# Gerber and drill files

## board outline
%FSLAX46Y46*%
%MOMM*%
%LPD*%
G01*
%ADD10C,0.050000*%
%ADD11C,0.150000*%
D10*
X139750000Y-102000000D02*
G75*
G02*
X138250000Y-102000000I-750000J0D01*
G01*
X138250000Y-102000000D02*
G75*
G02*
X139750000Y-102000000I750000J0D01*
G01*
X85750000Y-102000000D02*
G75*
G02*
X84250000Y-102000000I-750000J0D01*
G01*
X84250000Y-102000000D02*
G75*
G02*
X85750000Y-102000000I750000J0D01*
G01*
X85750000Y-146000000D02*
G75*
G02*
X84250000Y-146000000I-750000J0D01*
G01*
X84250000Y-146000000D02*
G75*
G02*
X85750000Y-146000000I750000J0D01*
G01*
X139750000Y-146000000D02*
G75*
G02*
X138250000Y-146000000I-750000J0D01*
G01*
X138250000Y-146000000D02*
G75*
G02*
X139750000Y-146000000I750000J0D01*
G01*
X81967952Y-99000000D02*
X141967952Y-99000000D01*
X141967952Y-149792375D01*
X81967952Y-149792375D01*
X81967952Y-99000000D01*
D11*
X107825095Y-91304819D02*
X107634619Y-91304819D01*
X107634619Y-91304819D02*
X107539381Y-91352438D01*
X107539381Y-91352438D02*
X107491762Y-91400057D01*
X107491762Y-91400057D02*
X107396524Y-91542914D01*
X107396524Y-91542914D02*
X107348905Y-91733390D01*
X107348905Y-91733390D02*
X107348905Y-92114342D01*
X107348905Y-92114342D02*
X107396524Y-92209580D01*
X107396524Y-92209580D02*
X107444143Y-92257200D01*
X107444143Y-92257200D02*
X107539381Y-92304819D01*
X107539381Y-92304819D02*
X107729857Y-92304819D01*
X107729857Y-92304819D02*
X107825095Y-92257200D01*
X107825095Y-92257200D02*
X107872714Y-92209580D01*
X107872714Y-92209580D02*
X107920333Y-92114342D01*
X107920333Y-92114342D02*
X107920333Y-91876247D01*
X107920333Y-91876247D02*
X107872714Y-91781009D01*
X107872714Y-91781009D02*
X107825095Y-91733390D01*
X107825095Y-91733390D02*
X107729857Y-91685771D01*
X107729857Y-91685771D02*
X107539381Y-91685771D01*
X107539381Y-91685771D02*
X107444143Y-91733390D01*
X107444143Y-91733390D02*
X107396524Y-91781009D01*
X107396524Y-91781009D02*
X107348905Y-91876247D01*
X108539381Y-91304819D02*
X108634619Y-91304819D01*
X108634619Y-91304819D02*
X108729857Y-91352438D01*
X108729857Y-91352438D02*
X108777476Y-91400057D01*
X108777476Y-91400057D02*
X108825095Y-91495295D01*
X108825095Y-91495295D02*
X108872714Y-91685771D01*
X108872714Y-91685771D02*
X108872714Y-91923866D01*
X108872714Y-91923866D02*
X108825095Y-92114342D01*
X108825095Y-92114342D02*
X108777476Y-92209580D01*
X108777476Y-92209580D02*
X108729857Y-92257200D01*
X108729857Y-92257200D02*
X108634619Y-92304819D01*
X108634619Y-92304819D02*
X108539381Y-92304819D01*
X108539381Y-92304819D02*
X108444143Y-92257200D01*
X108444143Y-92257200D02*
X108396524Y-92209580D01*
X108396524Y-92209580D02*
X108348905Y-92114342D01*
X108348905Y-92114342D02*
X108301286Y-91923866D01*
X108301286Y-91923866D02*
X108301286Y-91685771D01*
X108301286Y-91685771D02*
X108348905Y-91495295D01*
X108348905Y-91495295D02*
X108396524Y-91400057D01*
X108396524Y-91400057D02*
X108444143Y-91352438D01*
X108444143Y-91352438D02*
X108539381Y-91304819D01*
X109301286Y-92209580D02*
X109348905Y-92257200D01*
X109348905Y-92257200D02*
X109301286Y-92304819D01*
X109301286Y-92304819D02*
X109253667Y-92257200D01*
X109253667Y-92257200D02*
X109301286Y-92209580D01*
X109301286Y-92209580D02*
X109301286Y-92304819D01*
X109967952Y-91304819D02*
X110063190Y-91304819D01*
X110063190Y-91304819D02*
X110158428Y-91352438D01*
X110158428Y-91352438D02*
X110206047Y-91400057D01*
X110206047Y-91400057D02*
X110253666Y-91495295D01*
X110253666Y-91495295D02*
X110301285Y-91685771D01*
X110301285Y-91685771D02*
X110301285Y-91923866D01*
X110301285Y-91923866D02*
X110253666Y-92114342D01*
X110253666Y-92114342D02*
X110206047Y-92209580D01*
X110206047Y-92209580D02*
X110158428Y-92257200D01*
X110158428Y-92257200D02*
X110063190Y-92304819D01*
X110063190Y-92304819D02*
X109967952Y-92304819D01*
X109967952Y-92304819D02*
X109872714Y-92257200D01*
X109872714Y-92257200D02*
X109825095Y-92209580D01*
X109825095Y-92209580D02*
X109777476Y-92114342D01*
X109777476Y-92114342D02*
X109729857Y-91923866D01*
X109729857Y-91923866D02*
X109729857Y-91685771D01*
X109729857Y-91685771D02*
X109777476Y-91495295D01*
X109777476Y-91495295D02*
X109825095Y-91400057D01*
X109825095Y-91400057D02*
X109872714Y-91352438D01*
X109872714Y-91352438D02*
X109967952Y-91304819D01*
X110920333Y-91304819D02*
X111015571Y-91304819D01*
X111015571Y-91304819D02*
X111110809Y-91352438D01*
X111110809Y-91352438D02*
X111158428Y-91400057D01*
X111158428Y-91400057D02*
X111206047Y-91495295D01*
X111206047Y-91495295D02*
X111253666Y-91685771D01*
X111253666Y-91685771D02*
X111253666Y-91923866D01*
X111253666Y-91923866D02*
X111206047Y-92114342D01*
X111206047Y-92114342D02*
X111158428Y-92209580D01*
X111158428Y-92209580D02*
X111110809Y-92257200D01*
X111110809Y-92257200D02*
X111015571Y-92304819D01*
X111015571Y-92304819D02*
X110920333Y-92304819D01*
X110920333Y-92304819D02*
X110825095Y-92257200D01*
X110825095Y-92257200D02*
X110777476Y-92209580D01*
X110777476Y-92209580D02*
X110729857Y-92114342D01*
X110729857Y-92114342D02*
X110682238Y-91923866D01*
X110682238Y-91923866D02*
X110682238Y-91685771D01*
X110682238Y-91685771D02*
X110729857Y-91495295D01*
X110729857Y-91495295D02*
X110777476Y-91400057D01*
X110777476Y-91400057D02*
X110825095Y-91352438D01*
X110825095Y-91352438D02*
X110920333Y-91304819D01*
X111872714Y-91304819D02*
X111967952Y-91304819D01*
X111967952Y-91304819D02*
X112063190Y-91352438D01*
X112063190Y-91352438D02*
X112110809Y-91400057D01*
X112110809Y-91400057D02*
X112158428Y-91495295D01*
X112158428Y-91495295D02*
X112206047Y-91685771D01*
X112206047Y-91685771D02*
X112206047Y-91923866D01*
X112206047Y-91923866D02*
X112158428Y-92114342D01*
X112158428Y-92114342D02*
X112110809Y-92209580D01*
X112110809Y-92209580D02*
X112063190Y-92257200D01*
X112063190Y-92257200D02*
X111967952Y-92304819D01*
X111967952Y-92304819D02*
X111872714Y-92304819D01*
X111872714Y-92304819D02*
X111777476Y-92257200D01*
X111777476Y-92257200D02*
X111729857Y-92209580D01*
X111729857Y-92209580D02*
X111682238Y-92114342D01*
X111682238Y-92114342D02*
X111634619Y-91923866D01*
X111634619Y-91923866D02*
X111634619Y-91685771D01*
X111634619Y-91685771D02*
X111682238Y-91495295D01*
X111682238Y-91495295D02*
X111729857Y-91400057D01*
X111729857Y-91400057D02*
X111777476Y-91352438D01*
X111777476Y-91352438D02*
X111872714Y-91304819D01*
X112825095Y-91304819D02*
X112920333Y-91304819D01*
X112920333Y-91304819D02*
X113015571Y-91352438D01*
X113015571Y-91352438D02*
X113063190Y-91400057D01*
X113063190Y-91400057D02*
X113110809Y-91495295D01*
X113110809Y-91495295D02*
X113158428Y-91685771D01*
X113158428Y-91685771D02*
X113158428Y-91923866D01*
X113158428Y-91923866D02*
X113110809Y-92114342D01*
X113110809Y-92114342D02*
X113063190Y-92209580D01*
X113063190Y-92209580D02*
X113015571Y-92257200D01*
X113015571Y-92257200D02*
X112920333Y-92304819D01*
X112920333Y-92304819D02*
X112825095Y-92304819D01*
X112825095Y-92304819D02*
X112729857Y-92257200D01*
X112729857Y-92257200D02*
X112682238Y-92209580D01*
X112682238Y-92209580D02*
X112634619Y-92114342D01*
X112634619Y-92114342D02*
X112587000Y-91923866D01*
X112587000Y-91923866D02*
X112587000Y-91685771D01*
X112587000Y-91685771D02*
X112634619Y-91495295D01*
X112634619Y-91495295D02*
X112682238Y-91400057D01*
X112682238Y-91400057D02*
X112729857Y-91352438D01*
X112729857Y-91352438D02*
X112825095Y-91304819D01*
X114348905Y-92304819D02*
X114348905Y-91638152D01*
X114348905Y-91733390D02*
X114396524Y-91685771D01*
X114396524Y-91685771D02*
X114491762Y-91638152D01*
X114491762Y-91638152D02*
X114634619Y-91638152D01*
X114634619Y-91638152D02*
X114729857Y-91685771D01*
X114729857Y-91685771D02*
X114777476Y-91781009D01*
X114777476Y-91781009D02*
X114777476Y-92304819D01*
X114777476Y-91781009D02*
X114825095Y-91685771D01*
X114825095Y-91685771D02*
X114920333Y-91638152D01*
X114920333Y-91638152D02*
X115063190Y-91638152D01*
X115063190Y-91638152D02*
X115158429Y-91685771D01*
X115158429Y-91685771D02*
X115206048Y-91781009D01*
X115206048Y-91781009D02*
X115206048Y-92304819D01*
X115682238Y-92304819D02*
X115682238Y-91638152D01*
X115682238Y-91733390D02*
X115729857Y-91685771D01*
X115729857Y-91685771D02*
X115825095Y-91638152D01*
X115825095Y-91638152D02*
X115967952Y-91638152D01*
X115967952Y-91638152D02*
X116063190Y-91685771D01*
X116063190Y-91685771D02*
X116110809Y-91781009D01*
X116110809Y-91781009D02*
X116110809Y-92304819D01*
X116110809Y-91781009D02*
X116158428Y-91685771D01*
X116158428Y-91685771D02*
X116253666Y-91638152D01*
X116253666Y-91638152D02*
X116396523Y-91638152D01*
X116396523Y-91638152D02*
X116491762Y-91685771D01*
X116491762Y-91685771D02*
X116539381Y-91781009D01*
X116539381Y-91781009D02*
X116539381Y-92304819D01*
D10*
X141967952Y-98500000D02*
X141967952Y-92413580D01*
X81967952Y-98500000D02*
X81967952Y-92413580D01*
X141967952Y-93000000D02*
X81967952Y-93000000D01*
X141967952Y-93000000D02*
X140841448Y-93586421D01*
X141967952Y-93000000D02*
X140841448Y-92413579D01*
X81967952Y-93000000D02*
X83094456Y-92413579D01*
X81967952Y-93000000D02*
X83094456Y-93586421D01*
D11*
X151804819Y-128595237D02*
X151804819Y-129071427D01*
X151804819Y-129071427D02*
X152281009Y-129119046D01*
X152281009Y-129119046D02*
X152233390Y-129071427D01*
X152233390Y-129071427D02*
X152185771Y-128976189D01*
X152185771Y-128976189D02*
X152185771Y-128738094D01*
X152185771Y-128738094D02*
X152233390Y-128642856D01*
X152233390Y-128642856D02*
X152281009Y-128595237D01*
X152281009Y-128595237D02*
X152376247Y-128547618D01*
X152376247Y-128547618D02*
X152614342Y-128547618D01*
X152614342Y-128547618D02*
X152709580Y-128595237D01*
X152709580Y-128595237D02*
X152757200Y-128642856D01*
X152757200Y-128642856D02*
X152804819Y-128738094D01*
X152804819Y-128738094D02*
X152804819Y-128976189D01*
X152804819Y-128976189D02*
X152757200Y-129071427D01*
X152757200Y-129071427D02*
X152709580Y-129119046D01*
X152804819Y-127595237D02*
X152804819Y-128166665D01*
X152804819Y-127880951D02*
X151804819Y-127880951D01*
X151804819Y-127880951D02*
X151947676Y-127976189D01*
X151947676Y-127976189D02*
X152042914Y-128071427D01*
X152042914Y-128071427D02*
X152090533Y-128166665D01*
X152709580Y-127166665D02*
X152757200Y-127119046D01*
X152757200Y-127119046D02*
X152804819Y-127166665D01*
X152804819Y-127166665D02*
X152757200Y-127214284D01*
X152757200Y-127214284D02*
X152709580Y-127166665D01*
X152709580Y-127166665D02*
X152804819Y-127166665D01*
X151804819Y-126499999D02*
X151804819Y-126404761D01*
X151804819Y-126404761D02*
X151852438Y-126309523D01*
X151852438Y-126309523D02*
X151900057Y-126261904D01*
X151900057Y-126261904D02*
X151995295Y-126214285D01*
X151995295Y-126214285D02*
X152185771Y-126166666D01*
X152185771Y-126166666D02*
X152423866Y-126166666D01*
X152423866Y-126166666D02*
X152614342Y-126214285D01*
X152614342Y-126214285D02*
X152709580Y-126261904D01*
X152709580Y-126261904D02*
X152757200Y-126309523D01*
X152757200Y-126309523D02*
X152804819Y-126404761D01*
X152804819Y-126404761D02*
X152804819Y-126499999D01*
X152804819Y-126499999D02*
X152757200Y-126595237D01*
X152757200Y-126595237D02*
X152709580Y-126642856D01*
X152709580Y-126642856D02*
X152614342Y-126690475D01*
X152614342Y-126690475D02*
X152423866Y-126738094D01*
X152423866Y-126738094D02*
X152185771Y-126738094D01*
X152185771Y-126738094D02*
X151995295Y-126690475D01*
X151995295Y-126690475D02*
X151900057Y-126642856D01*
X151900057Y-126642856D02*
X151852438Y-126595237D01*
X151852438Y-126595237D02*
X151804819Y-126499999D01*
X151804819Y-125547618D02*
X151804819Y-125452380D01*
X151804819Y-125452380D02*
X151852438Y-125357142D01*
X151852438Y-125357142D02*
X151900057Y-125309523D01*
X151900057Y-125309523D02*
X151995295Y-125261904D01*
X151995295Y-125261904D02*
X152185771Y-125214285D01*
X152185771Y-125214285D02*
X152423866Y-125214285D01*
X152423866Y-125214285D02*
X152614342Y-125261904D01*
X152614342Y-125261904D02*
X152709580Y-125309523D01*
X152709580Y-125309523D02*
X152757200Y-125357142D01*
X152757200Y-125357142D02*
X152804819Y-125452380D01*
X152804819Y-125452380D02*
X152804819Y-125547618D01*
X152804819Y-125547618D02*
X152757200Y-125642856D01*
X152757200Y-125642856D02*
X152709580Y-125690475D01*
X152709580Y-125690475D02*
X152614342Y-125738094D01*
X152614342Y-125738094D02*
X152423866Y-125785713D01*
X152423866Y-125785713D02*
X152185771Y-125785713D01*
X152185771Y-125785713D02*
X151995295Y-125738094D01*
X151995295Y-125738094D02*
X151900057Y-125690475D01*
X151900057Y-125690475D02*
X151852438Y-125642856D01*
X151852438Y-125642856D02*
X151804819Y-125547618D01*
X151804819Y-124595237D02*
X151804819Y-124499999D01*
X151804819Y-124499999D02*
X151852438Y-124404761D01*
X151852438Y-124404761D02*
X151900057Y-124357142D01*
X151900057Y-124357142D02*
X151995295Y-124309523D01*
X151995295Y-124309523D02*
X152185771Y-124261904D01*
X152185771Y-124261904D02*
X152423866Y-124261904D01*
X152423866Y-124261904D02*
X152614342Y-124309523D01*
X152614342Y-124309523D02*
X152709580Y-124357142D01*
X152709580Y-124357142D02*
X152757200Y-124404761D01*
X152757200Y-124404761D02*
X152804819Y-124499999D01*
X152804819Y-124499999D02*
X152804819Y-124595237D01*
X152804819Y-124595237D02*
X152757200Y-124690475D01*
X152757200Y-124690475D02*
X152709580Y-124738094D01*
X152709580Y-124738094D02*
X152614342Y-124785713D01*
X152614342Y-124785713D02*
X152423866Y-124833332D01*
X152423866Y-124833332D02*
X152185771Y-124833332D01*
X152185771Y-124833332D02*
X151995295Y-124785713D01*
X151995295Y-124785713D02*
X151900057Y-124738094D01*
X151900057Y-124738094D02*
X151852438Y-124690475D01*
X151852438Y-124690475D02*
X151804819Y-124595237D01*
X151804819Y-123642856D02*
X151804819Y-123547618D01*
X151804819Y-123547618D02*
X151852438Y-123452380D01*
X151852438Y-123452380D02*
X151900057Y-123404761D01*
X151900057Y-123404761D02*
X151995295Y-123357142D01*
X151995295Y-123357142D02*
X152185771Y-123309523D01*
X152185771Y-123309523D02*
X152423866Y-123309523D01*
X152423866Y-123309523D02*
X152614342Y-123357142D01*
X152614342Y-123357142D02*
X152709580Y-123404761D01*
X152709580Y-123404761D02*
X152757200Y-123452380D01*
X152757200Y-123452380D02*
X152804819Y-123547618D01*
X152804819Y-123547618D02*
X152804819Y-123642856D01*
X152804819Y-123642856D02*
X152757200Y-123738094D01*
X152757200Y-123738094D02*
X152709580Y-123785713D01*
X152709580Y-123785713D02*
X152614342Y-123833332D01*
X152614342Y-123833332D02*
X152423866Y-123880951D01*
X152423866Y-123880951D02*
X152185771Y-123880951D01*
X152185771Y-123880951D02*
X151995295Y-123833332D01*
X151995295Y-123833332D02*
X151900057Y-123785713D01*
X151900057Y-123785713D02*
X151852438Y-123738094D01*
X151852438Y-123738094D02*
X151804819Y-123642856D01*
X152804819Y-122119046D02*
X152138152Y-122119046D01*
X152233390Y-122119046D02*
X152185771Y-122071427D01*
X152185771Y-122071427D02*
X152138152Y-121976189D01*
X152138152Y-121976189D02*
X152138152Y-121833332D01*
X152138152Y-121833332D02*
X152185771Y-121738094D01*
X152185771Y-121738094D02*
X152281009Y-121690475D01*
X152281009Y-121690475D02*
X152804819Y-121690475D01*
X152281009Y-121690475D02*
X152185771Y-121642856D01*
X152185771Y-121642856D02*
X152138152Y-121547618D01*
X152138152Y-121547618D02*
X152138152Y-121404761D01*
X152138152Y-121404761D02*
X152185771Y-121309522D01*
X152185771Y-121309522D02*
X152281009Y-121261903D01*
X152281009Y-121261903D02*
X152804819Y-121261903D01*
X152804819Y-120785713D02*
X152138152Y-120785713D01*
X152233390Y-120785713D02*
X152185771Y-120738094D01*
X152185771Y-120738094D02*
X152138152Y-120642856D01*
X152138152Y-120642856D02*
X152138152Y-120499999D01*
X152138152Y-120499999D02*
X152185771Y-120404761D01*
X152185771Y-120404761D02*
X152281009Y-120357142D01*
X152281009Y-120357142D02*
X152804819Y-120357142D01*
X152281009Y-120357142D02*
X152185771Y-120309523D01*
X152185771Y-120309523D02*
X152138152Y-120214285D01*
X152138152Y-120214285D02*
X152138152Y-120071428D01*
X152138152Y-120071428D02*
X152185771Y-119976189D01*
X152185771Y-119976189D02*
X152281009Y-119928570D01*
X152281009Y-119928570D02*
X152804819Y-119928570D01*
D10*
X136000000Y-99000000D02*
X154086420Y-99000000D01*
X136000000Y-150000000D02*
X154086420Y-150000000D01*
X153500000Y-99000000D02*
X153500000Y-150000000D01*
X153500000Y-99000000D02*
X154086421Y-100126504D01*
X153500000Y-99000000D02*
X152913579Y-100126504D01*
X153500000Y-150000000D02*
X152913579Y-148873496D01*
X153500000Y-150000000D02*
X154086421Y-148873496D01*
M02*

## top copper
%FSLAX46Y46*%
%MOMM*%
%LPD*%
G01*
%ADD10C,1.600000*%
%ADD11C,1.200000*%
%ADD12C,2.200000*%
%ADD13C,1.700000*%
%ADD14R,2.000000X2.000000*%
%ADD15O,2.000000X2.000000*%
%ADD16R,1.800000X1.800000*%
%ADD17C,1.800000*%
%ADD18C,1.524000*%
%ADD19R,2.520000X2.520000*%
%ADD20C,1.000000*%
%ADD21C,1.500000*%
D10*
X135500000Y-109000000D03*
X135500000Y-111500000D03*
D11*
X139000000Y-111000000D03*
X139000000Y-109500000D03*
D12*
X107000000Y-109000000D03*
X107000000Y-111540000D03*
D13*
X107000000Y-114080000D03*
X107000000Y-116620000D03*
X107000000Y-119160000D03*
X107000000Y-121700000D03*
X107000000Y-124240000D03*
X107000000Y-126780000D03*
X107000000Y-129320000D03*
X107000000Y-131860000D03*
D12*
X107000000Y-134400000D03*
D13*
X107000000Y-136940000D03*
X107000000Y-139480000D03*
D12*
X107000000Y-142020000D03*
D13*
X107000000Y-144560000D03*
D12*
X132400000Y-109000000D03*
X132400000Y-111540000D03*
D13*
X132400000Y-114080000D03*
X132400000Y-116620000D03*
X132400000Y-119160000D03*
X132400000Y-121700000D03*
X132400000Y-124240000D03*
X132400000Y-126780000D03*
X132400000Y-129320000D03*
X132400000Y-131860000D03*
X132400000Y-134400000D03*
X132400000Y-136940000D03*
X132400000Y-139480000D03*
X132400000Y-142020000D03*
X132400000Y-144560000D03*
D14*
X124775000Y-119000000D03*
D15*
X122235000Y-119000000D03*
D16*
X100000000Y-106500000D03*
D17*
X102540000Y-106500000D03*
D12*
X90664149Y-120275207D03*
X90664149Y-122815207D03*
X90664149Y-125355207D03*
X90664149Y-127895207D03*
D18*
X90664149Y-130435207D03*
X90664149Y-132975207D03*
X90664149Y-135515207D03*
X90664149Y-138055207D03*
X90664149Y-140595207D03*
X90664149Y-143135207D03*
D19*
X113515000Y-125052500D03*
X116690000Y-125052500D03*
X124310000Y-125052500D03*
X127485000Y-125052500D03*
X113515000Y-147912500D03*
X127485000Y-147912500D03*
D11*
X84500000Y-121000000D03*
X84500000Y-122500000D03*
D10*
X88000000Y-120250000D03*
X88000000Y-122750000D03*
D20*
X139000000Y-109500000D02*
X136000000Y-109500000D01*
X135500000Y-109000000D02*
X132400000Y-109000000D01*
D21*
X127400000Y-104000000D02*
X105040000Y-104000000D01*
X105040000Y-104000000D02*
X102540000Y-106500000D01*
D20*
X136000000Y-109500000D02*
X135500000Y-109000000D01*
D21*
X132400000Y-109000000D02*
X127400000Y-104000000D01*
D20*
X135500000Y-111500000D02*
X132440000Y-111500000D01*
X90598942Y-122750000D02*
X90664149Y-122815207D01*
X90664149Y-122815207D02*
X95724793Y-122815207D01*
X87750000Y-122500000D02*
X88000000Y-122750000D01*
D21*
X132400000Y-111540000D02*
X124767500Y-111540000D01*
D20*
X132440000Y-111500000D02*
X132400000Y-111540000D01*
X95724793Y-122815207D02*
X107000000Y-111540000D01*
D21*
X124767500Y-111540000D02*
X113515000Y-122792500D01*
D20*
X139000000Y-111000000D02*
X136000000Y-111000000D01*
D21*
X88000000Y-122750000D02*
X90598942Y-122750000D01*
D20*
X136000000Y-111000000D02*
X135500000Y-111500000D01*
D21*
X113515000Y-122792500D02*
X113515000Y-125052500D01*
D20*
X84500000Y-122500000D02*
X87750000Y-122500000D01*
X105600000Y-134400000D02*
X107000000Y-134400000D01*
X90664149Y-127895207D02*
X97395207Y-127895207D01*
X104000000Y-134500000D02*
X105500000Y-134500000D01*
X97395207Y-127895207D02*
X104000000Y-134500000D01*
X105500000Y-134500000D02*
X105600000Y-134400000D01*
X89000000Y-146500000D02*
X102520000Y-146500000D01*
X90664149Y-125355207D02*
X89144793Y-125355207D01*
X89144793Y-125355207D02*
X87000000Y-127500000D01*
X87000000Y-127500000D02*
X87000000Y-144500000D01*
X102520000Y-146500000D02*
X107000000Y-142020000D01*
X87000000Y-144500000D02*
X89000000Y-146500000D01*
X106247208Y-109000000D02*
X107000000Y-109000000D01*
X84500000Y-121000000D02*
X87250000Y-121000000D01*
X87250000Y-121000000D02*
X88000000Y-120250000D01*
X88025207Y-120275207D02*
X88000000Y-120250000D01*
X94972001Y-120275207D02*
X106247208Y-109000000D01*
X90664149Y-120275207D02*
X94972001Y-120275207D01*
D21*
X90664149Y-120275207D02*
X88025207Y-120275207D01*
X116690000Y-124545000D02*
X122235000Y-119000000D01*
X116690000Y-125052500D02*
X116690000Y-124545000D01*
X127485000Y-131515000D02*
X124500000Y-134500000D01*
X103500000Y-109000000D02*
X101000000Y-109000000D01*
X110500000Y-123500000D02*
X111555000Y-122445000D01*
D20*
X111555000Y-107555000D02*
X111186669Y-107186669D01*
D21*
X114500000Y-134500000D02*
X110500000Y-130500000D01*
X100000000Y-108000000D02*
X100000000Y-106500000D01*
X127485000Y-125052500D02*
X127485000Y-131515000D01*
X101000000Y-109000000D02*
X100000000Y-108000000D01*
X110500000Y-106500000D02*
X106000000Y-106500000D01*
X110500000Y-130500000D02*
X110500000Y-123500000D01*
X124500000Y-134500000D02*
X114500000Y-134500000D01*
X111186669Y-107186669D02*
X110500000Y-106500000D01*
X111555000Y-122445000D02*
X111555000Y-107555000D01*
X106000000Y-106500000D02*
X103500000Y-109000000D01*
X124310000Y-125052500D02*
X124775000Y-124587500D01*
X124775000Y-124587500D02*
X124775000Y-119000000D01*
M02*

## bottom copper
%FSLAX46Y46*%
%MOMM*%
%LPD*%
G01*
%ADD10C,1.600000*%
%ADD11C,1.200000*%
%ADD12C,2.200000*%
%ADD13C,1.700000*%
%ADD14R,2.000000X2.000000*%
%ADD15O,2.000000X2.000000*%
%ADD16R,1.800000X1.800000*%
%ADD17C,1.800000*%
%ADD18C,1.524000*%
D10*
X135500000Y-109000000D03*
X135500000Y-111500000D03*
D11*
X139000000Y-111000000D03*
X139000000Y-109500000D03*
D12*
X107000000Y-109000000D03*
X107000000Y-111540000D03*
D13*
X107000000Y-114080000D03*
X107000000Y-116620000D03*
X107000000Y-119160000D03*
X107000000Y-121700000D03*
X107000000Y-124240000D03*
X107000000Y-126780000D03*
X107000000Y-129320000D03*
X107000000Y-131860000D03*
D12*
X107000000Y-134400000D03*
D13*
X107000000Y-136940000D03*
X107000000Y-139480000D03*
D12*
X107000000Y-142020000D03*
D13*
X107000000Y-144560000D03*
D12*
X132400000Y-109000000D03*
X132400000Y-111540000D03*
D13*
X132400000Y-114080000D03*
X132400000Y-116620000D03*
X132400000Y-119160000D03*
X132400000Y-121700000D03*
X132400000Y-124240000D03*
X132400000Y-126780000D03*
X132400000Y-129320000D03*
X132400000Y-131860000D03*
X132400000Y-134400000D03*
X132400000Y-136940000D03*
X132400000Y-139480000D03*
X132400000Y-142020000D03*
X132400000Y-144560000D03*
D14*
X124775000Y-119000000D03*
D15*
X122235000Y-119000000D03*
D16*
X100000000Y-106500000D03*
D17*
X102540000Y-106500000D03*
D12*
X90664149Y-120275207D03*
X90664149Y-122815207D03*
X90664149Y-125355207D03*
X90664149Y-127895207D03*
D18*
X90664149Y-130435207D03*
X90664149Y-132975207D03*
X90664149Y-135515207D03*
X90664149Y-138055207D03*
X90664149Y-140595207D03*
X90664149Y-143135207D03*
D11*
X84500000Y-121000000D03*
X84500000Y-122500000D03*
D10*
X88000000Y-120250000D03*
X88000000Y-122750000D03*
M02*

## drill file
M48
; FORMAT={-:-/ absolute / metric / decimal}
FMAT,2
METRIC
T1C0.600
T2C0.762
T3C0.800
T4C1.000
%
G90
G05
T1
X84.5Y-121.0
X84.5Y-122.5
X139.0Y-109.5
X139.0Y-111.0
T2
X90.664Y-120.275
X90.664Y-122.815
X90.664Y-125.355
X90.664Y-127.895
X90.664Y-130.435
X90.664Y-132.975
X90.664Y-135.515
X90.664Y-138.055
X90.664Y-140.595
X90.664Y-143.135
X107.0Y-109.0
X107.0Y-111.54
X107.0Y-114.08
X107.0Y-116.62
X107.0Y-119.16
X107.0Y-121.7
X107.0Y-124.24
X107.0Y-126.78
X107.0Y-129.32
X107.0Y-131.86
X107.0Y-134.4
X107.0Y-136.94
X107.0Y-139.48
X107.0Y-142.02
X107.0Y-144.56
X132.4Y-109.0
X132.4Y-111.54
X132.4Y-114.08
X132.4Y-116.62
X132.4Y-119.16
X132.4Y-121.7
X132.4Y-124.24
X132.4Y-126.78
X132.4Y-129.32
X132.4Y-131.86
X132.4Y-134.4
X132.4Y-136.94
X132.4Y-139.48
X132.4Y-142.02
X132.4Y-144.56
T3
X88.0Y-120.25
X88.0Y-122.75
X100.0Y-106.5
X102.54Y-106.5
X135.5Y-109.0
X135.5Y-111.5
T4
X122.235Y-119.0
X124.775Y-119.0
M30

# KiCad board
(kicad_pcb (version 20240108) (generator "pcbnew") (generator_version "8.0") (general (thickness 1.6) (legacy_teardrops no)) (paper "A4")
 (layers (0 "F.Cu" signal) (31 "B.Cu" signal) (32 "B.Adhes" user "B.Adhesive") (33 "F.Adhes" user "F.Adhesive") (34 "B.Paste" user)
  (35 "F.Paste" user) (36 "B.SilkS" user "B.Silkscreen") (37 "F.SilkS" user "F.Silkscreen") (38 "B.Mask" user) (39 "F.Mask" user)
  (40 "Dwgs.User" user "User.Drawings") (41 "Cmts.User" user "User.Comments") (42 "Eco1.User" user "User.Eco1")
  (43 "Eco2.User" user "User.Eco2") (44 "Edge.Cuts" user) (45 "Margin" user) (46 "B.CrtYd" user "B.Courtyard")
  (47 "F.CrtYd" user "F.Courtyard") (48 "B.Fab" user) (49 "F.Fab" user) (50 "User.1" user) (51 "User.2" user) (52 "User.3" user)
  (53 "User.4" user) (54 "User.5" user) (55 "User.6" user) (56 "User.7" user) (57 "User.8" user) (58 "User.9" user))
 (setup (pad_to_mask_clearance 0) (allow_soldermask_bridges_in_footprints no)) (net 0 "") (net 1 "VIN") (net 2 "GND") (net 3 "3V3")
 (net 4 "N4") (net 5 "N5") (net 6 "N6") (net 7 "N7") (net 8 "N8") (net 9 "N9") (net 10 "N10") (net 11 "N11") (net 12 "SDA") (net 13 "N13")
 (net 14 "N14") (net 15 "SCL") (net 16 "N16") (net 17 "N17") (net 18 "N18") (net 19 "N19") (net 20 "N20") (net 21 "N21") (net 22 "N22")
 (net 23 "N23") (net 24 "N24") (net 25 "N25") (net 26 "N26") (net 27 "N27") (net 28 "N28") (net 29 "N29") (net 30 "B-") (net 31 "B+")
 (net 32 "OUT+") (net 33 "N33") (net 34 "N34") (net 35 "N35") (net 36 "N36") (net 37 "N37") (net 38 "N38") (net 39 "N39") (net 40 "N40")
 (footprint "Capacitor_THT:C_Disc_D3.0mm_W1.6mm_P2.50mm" (layer "F.Cu") (at 135.5 109 -90)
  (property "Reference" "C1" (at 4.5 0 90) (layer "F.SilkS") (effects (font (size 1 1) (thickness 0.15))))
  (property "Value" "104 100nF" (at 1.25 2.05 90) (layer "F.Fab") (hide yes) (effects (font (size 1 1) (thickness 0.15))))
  (pad "1" thru_hole circle (at 0 0 270) (size 1.6 1.6) (drill 0.8) (layers "*.Cu" "*.Mask") (remove_unused_layers no) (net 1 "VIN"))
  (pad "2" thru_hole circle (at 2.5 0 270) (size 1.6 1.6) (drill 0.8) (layers "*.Cu" "*.Mask") (remove_unused_layers no) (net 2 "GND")))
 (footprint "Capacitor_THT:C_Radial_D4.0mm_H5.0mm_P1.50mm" (layer "F.Cu") (at 139 109.5 -90)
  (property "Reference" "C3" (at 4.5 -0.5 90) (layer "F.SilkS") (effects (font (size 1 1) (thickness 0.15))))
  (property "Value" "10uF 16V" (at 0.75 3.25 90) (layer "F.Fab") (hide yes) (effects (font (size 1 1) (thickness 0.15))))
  (pad "2" thru_hole circle (at 1.5 0 270) (size 1.2 1.2) (drill 0.6) (layers "*.Cu" "*.Mask") (remove_unused_layers no) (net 2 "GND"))
  (pad "E" thru_hole circle (at 0 0 270) (size 1.2 1.2) (drill 0.6) (layers "*.Cu" "*.Mask") (remove_unused_layers no) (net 1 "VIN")))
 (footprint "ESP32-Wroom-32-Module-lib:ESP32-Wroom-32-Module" (layer "F.Cu") (at 107 101.38)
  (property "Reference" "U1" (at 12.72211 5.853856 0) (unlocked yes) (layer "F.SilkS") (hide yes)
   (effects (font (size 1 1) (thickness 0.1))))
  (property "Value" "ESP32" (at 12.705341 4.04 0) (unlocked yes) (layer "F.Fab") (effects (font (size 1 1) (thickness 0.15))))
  (pad "1" thru_hole circle (at 0 7.62) (size 2.2 2.2) (drill 0.762) (layers "*.Cu" "*.Mask") (remove_unused_layers no) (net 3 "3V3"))
  (pad "2" thru_hole circle (at 0 10.16) (size 2.2 2.2) (drill 0.762) (layers "*.Cu" "*.Mask") (remove_unused_layers no) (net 2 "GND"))
  (pad "3" thru_hole circle (at 0 12.7) (size 1.7 1.7) (drill 0.762) (layers "*.Cu" "*.Mask") (remove_unused_layers no) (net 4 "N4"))
  (pad "4" thru_hole circle (at 0 15.24) (size 1.7 1.7) (drill 0.762) (layers "*.Cu" "*.Mask") (remove_unused_layers no) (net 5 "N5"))
  (pad "5" thru_hole circle (at 0 17.78) (size 1.7 1.7) (drill 0.762) (layers "*.Cu" "*.Mask") (remove_unused_layers no) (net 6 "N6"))
  (pad "6" thru_hole circle (at 0 20.32) (size 1.7 1.7) (drill 0.762) (layers "*.Cu" "*.Mask") (remove_unused_layers no) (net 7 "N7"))
  (pad "7" thru_hole circle (at 0 22.86) (size 1.7 1.7) (drill 0.762) (layers "*.Cu" "*.Mask") (remove_unused_layers no) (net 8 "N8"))
  (pad "8" thru_hole circle (at 0 25.4) (size 1.7 1.7) (drill 0.762) (layers "*.Cu" "*.Mask") (remove_unused_layers no) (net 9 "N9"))
  (pad "9" thru_hole circle (at 0 27.94) (size 1.7 1.7) (drill 0.762) (layers "*.Cu" "*.Mask") (remove_unused_layers no) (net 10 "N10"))
  (pad "10" thru_hole circle (at 0 30.48) (size 1.7 1.7) (drill 0.762) (layers "*.Cu" "*.Mask") (remove_unused_layers no) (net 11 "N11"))
  (pad "11" thru_hole circle (at 0 33.02) (size 2.2 2.2) (drill 0.762) (layers "*.Cu" "*.Mask") (remove_unused_layers no) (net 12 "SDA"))
  (pad "12" thru_hole circle (at 0 35.56) (size 1.7 1.7) (drill 0.762) (layers "*.Cu" "*.Mask") (remove_unused_layers no) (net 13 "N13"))
  (pad "13" thru_hole circle (at 0 38.1) (size 1.7 1.7) (drill 0.762) (layers "*.Cu" "*.Mask") (remove_unused_layers no) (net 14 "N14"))
  (pad "14" thru_hole circle (at 0 40.64) (size 2.2 2.2) (drill 0.762) (layers "*.Cu" "*.Mask") (remove_unused_layers no) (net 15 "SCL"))
  (pad "15" thru_hole circle (at 0 43.18) (size 1.7 1.7) (drill 0.762) (layers "*.Cu" "*.Mask") (remove_unused_layers no) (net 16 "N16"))
  (pad "16" thru_hole circle (at 25.4 7.62) (size 2.2 2.2) (drill 0.762) (layers "*.Cu" "*.Mask") (remove_unused_layers no) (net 1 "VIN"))
  (pad "17" thru_hole circle (at 25.4 10.16) (size 2.2 2.2) (drill 0.762) (layers "*.Cu" "*.Mask") (remove_unused_layers no) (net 2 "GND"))
  (pad "18" thru_hole circle (at 25.4 12.7) (size 1.7 1.7) (drill 0.762) (layers "*.Cu" "*.Mask") (remove_unused_layers no) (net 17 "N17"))
  (pad "19" thru_hole circle (at 25.4 15.24) (size 1.7 1.7) (drill 0.762) (layers "*.Cu" "*.Mask") (remove_unused_layers no) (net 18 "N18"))
  (pad "20" thru_hole circle (at 25.4 17.78) (size 1.7 1.7) (drill 0.762) (layers "*.Cu" "*.Mask") (remove_unused_layers no) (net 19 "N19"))
  (pad "21" thru_hole circle (at 25.4 20.32) (size 1.7 1.7) (drill 0.762) (layers "*.Cu" "*.Mask") (remove_unused_layers no) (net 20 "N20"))
  (pad "22" thru_hole circle (at 25.4 22.86) (size 1.7 1.7) (drill 0.762) (layers "*.Cu" "*.Mask") (remove_unused_layers no) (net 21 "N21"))
  (pad "23" thru_hole circle (at 25.4 25.4) (size 1.7 1.7) (drill 0.762) (layers "*.Cu" "*.Mask") (remove_unused_layers no) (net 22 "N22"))
  (pad "24" thru_hole circle (at 25.4 27.94) (size 1.7 1.7) (drill 0.762) (layers "*.Cu" "*.Mask") (remove_unused_layers no) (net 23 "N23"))
  (pad "25" thru_hole circle (at 25.4 30.48) (size 1.7 1.7) (drill 0.762) (layers "*.Cu" "*.Mask") (remove_unused_layers no) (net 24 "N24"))
  (pad "26" thru_hole circle (at 25.4 33.02) (size 1.7 1.7) (drill 0.762) (layers "*.Cu" "*.Mask") (remove_unused_layers no) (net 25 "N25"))
  (pad "27" thru_hole circle (at 25.4 35.56) (size 1.7 1.7) (drill 0.762) (layers "*.Cu" "*.Mask") (remove_unused_layers no) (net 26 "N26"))
  (pad "28" thru_hole circle (at 25.4 38.1) (size 1.7 1.7) (drill 0.762) (layers "*.Cu" "*.Mask") (remove_unused_layers no) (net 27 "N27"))
  (pad "29" thru_hole circle (at 25.4 40.64) (size 1.7 1.7) (drill 0.762) (layers "*.Cu" "*.Mask") (remove_unused_layers no) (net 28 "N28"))
  (pad "30" thru_hole circle (at 25.4 43.18) (size 1.7 1.7) (drill 0.762) (layers "*.Cu" "*.Mask") (remove_unused_layers no) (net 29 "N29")))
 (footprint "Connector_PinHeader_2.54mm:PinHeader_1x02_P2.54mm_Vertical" (layer "F.Cu") (at 124.775 119 -90)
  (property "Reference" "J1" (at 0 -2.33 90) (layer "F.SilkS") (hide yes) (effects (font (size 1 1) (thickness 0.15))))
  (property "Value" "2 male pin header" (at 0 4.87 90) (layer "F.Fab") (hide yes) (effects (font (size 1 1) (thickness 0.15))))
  (pad "1" thru_hole rect (at 0 0 270) (size 2 2) (drill 1) (layers "*.Cu" "*.Mask") (remove_unused_layers no) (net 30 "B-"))
  (pad "2" thru_hole oval (at 0 2.54 270) (size 2 2) (drill 1) (layers "*.Cu" "*.Mask") (remove_unused_layers no) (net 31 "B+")))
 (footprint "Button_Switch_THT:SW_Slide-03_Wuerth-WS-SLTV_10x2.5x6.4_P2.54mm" (layer "F.Cu") (at 100 106.5 180)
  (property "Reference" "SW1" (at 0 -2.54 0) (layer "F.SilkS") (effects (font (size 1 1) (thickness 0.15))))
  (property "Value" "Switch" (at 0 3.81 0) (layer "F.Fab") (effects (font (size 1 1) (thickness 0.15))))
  (pad "1" thru_hole rect (at 0 0 180) (size 1.8 1.8) (drill 0.8) (layers "*.Cu" "*.Mask") (remove_unused_layers no) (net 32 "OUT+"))
  (pad "2" thru_hole circle (at -2.54 0 180) (size 1.8 1.8) (drill 0.8) (layers "*.Cu" "*.Mask") (remove_unused_layers no) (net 1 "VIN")))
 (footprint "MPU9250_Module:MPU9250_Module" (layer "F.Cu") (at 97 114.5)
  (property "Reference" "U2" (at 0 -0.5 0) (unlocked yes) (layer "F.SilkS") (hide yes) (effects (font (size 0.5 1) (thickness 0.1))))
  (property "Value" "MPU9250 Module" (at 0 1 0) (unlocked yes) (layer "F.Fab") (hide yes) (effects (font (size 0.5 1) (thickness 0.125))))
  (pad "1" thru_hole circle (at -6.335851 5.775207) (size 2.2 2.2) (drill 0.762) (layers "*.Cu" "*.Mask") (remove_unused_layers no)
   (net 3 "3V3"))
  (pad "2" thru_hole circle (at -6.335851 8.315207) (size 2.2 2.2) (drill 0.762) (layers "*.Cu" "*.Mask") (remove_unused_layers no)
   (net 2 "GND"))
  (pad "3" thru_hole circle (at -6.335851 10.855207) (size 2.2 2.2) (drill 0.762) (layers "*.Cu" "*.Mask") (remove_unused_layers no)
   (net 15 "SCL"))
  (pad "4" thru_hole circle (at -6.335851 13.395207) (size 2.2 2.2) (drill 0.762) (layers "*.Cu" "*.Mask") (remove_unused_layers no)
   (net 12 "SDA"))
  (pad "5" thru_hole circle (at -6.335851 15.935207) (size 1.524 1.524) (drill 0.762) (layers "*.Cu" "*.Mask") (remove_unused_layers no)
   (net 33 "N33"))
  (pad "6" thru_hole circle (at -6.335851 18.475207) (size 1.524 1.524) (drill 0.762) (layers "*.Cu" "*.Mask") (remove_unused_layers no)
   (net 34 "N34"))
  (pad "7" thru_hole circle (at -6.335851 21.015207) (size 1.524 1.524) (drill 0.762) (layers "*.Cu" "*.Mask") (remove_unused_layers no)
   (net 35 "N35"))
  (pad "8" thru_hole circle (at -6.335851 23.555207) (size 1.524 1.524) (drill 0.762) (layers "*.Cu" "*.Mask") (remove_unused_layers no)
   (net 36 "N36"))
  (pad "9" thru_hole circle (at -6.335851 26.095207) (size 1.524 1.524) (drill 0.762) (layers "*.Cu" "*.Mask") (remove_unused_layers no)
   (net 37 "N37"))
  (pad "10" thru_hole circle (at -6.335851 28.635207) (size 1.524 1.524) (drill 0.762) (layers "*.Cu" "*.Mask") (remove_unused_layers no)
   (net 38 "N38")))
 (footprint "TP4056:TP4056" (layer "F.Cu") (at 120.5 116.7475)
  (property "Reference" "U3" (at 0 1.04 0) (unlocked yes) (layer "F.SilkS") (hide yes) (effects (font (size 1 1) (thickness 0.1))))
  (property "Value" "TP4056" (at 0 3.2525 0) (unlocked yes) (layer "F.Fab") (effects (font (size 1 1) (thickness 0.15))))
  (pad "1" smd rect (at -6.985 8.305 90) (size 2.52 2.52) (layers "F.Cu" "F.Paste" "F.Mask") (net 2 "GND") (thermal_bridge_angle 45))
  (pad "2" smd rect (at -3.81 8.305 90) (size 2.52 2.52) (layers "F.Cu" "F.Paste" "F.Mask") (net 31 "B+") (thermal_bridge_angle 45))
  (pad "3" smd rect (at 3.81 8.305 90) (size 2.52 2.52) (layers "F.Cu" "F.Paste" "F.Mask") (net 30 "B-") (thermal_bridge_angle 45))
  (pad "4" smd rect (at 6.985 8.305 90) (size 2.52 2.52) (layers "F.Cu" "F.Paste" "F.Mask") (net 32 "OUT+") (thermal_bridge_angle 45))
  (pad "5" smd rect (at -6.985 31.165 90) (size 2.52 2.52) (layers "F.Cu" "F.Paste" "F.Mask") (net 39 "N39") (thermal_bridge_angle 45))
  (pad "6" smd rect (at 6.985 31.165 90) (size 2.52 2.52) (layers "F.Cu" "F.Paste" "F.Mask") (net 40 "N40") (thermal_bridge_angle 45)))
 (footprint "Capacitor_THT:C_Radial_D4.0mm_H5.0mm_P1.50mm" (layer "F.Cu") (at 84.5 121 -90)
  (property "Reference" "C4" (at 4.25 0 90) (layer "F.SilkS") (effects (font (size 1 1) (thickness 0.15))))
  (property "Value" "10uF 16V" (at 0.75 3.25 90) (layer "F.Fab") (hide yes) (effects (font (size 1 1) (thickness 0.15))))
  (pad "1" thru_hole circle (at 0 0 270) (size 1.2 1.2) (drill 0.6) (layers "*.Cu" "*.Mask") (remove_unused_layers no) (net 3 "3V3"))
  (pad "2" thru_hole circle (at 1.5 0 270) (size 1.2 1.2) (drill 0.6) (layers "*.Cu" "*.Mask") (remove_unused_layers no) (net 2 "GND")))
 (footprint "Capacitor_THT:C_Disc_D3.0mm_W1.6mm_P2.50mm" (layer "F.Cu") (at 88 120.25 -90)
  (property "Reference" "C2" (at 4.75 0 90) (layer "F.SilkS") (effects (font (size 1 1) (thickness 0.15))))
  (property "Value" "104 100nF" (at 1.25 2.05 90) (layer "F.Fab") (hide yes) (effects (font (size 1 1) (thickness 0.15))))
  (pad "1" thru_hole circle (at 0 0 270) (size 1.6 1.6) (drill 0.8) (layers "*.Cu" "*.Mask") (remove_unused_layers no) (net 3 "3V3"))
  (pad "2" thru_hole circle (at 2.5 0 270) (size 1.6 1.6) (drill 0.8) (layers "*.Cu" "*.Mask") (remove_unused_layers no) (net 2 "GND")))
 (gr_circle (center 139 102) (end 139.75 102) (stroke (width 0.05) (type default)) (fill none) (layer "Edge.Cuts"))
 (gr_circle (center 85 102) (end 85.75 102) (stroke (width 0.05) (type default)) (fill none) (layer "Edge.Cuts"))
 (gr_circle (center 85 146) (end 85.75 146) (stroke (width 0.05) (type default)) (fill none) (layer "Edge.Cuts"))
 (gr_circle (center 139 146) (end 139.75 146) (stroke (width 0.05) (type default)) (fill none) (layer "Edge.Cuts"))
 (gr_rect (start 81.967952 99) (end 141.967952 149.792375) (stroke (width 0.05) (type default)) (fill none) (layer "Edge.Cuts"))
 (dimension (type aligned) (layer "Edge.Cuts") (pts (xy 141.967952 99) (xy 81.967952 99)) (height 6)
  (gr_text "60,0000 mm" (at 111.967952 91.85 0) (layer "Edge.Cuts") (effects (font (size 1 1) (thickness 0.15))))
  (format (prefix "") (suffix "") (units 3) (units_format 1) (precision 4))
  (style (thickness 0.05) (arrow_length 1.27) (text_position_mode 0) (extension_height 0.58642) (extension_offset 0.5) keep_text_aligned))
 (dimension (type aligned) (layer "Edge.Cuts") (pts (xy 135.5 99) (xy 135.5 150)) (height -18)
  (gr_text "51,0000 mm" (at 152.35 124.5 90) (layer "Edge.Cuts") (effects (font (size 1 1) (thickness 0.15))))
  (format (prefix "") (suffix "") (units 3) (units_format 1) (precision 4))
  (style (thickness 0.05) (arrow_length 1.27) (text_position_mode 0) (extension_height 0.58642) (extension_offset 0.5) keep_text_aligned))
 (segment (start 139 109.5) (end 136 109.5) (width 1) (layer "F.Cu") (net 1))
 (segment (start 135.5 109) (end 132.4 109) (width 1) (layer "F.Cu") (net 1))
 (segment (start 127.4 104) (end 105.04 104) (width 1.5) (layer "F.Cu") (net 1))
 (segment (start 105.04 104) (end 102.54 106.5) (width 1.5) (layer "F.Cu") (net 1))
 (segment (start 136 109.5) (end 135.5 109) (width 1) (layer "F.Cu") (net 1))
 (segment (start 132.4 109) (end 127.4 104) (width 1.5) (layer "F.Cu") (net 1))
 (segment (start 135.5 111.5) (end 132.44 111.5) (width 1) (layer "F.Cu") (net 2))
 (segment (start 90.598942 122.75) (end 90.664149 122.815207) (width 1) (layer "F.Cu") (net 2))
 (segment (start 90.664149 122.815207) (end 95.724793 122.815207) (width 1) (layer "F.Cu") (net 2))
 (segment (start 87.75 122.5) (end 88 122.75) (width 1) (layer "F.Cu") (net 2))
 (segment (start 132.4 111.54) (end 124.7675 111.54) (width 1.5) (layer "F.Cu") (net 2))
 (segment (start 132.44 111.5) (end 132.4 111.54) (width 1) (layer "F.Cu") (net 2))
 (segment (start 95.724793 122.815207) (end 107 111.54) (width 1) (layer "F.Cu") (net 2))
 (segment (start 124.7675 111.54) (end 113.515 122.7925) (width 1.5) (layer "F.Cu") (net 2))
 (segment (start 139 111) (end 136 111) (width 1) (layer "F.Cu") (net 2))
 (segment (start 88 122.75) (end 90.598942 122.75) (width 1.5) (layer "F.Cu") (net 2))
 (segment (start 136 111) (end 135.5 111.5) (width 1) (layer "F.Cu") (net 2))
 (segment (start 113.515 122.7925) (end 113.515 125.0525) (width 1.5) (layer "F.Cu") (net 2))
 (segment (start 84.5 122.5) (end 87.75 122.5) (width 1) (layer "F.Cu") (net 2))
 (segment (start 105.6 134.4) (end 107 134.4) (width 1) (layer "F.Cu") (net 12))
 (segment (start 90.664149 127.895207) (end 97.395207 127.895207) (width 1) (layer "F.Cu") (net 12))
 (segment (start 104 134.5) (end 105.5 134.5) (width 1) (layer "F.Cu") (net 12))
 (segment (start 97.395207 127.895207) (end 104 134.5) (width 1) (layer "F.Cu") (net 12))
 (segment (start 105.5 134.5) (end 105.6 134.4) (width 1) (layer "F.Cu") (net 12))
 (segment (start 89 146.5) (end 102.52 146.5) (width 1) (layer "F.Cu") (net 15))
 (segment (start 90.664149 125.355207) (end 89.144793 125.355207) (width 1) (layer "F.Cu") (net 15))
 (segment (start 89.144793 125.355207) (end 87 127.5) (width 1) (layer "F.Cu") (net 15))
 (segment (start 87 127.5) (end 87 144.5) (width 1) (layer "F.Cu") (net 15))
 (segment (start 102.52 146.5) (end 107 142.02) (width 1) (layer "F.Cu") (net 15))
 (segment (start 87 144.5) (end 89 146.5) (width 1) (layer "F.Cu") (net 15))
 (segment (start 106.247208 109) (end 107 109) (width 1) (layer "F.Cu") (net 3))
 (segment (start 84.5 121) (end 87.25 121) (width 1) (layer "F.Cu") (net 3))
 (segment (start 87.25 121) (end 88 120.25) (width 1) (layer "F.Cu") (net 3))
 (segment (start 88.025207 120.275207) (end 88 120.25) (width 1) (layer "F.Cu") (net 3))
 (segment (start 94.972001 120.275207) (end 106.247208 109) (width 1) (layer "F.Cu") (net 3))
 (segment (start 90.664149 120.275207) (end 94.972001 120.275207) (width 1) (layer "F.Cu") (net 3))
 (segment (start 90.664149 120.275207) (end 88.025207 120.275207) (width 1.5) (layer "F.Cu") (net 3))
 (segment (start 116.69 124.545) (end 122.235 119) (width 1.5) (layer "F.Cu") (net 31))
 (segment (start 116.69 125.0525) (end 116.69 124.545) (width 1.5) (layer "F.Cu") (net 31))
 (segment (start 127.485 131.515) (end 124.5 134.5) (width 1.5) (layer "F.Cu") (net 32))
 (segment (start 103.5 109) (end 101 109) (width 1.5) (layer "F.Cu") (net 32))
 (segment (start 110.5 123.5) (end 111.555 122.445) (width 1.5) (layer "F.Cu") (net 32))
 (segment (start 111.555 107.555) (end 111.186669 107.186669) (width 1) (layer "F.Cu") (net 32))
 (segment (start 114.5 134.5) (end 110.5 130.5) (width 1.5) (layer "F.Cu") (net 32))
 (segment (start 100 108) (end 100 106.5) (width 1.5) (layer "F.Cu") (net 32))
 (segment (start 127.485 125.0525) (end 127.485 131.515) (width 1.5) (layer "F.Cu") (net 32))
 (segment (start 101 109) (end 100 108) (width 1.5) (layer "F.Cu") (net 32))
 (segment (start 110.5 106.5) (end 106 106.5) (width 1.5) (layer "F.Cu") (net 32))
 (segment (start 110.5 130.5) (end 110.5 123.5) (width 1.5) (layer "F.Cu") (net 32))
 (segment (start 124.5 134.5) (end 114.5 134.5) (width 1.5) (layer "F.Cu") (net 32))
 (segment (start 111.186669 107.186669) (end 110.5 106.5) (width 1.5) (layer "F.Cu") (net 32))
 (segment (start 111.555 122.445) (end 111.555 107.555) (width 1.5) (layer "F.Cu") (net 32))
 (segment (start 106 106.5) (end 103.5 109) (width 1.5) (layer "F.Cu") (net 32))
 (segment (start 124.31 125.0525) (end 124.775 124.5875) (width 1.5) (layer "F.Cu") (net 30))
 (segment (start 124.775 124.5875) (end 124.775 119) (width 1.5) (layer "F.Cu") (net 30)))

